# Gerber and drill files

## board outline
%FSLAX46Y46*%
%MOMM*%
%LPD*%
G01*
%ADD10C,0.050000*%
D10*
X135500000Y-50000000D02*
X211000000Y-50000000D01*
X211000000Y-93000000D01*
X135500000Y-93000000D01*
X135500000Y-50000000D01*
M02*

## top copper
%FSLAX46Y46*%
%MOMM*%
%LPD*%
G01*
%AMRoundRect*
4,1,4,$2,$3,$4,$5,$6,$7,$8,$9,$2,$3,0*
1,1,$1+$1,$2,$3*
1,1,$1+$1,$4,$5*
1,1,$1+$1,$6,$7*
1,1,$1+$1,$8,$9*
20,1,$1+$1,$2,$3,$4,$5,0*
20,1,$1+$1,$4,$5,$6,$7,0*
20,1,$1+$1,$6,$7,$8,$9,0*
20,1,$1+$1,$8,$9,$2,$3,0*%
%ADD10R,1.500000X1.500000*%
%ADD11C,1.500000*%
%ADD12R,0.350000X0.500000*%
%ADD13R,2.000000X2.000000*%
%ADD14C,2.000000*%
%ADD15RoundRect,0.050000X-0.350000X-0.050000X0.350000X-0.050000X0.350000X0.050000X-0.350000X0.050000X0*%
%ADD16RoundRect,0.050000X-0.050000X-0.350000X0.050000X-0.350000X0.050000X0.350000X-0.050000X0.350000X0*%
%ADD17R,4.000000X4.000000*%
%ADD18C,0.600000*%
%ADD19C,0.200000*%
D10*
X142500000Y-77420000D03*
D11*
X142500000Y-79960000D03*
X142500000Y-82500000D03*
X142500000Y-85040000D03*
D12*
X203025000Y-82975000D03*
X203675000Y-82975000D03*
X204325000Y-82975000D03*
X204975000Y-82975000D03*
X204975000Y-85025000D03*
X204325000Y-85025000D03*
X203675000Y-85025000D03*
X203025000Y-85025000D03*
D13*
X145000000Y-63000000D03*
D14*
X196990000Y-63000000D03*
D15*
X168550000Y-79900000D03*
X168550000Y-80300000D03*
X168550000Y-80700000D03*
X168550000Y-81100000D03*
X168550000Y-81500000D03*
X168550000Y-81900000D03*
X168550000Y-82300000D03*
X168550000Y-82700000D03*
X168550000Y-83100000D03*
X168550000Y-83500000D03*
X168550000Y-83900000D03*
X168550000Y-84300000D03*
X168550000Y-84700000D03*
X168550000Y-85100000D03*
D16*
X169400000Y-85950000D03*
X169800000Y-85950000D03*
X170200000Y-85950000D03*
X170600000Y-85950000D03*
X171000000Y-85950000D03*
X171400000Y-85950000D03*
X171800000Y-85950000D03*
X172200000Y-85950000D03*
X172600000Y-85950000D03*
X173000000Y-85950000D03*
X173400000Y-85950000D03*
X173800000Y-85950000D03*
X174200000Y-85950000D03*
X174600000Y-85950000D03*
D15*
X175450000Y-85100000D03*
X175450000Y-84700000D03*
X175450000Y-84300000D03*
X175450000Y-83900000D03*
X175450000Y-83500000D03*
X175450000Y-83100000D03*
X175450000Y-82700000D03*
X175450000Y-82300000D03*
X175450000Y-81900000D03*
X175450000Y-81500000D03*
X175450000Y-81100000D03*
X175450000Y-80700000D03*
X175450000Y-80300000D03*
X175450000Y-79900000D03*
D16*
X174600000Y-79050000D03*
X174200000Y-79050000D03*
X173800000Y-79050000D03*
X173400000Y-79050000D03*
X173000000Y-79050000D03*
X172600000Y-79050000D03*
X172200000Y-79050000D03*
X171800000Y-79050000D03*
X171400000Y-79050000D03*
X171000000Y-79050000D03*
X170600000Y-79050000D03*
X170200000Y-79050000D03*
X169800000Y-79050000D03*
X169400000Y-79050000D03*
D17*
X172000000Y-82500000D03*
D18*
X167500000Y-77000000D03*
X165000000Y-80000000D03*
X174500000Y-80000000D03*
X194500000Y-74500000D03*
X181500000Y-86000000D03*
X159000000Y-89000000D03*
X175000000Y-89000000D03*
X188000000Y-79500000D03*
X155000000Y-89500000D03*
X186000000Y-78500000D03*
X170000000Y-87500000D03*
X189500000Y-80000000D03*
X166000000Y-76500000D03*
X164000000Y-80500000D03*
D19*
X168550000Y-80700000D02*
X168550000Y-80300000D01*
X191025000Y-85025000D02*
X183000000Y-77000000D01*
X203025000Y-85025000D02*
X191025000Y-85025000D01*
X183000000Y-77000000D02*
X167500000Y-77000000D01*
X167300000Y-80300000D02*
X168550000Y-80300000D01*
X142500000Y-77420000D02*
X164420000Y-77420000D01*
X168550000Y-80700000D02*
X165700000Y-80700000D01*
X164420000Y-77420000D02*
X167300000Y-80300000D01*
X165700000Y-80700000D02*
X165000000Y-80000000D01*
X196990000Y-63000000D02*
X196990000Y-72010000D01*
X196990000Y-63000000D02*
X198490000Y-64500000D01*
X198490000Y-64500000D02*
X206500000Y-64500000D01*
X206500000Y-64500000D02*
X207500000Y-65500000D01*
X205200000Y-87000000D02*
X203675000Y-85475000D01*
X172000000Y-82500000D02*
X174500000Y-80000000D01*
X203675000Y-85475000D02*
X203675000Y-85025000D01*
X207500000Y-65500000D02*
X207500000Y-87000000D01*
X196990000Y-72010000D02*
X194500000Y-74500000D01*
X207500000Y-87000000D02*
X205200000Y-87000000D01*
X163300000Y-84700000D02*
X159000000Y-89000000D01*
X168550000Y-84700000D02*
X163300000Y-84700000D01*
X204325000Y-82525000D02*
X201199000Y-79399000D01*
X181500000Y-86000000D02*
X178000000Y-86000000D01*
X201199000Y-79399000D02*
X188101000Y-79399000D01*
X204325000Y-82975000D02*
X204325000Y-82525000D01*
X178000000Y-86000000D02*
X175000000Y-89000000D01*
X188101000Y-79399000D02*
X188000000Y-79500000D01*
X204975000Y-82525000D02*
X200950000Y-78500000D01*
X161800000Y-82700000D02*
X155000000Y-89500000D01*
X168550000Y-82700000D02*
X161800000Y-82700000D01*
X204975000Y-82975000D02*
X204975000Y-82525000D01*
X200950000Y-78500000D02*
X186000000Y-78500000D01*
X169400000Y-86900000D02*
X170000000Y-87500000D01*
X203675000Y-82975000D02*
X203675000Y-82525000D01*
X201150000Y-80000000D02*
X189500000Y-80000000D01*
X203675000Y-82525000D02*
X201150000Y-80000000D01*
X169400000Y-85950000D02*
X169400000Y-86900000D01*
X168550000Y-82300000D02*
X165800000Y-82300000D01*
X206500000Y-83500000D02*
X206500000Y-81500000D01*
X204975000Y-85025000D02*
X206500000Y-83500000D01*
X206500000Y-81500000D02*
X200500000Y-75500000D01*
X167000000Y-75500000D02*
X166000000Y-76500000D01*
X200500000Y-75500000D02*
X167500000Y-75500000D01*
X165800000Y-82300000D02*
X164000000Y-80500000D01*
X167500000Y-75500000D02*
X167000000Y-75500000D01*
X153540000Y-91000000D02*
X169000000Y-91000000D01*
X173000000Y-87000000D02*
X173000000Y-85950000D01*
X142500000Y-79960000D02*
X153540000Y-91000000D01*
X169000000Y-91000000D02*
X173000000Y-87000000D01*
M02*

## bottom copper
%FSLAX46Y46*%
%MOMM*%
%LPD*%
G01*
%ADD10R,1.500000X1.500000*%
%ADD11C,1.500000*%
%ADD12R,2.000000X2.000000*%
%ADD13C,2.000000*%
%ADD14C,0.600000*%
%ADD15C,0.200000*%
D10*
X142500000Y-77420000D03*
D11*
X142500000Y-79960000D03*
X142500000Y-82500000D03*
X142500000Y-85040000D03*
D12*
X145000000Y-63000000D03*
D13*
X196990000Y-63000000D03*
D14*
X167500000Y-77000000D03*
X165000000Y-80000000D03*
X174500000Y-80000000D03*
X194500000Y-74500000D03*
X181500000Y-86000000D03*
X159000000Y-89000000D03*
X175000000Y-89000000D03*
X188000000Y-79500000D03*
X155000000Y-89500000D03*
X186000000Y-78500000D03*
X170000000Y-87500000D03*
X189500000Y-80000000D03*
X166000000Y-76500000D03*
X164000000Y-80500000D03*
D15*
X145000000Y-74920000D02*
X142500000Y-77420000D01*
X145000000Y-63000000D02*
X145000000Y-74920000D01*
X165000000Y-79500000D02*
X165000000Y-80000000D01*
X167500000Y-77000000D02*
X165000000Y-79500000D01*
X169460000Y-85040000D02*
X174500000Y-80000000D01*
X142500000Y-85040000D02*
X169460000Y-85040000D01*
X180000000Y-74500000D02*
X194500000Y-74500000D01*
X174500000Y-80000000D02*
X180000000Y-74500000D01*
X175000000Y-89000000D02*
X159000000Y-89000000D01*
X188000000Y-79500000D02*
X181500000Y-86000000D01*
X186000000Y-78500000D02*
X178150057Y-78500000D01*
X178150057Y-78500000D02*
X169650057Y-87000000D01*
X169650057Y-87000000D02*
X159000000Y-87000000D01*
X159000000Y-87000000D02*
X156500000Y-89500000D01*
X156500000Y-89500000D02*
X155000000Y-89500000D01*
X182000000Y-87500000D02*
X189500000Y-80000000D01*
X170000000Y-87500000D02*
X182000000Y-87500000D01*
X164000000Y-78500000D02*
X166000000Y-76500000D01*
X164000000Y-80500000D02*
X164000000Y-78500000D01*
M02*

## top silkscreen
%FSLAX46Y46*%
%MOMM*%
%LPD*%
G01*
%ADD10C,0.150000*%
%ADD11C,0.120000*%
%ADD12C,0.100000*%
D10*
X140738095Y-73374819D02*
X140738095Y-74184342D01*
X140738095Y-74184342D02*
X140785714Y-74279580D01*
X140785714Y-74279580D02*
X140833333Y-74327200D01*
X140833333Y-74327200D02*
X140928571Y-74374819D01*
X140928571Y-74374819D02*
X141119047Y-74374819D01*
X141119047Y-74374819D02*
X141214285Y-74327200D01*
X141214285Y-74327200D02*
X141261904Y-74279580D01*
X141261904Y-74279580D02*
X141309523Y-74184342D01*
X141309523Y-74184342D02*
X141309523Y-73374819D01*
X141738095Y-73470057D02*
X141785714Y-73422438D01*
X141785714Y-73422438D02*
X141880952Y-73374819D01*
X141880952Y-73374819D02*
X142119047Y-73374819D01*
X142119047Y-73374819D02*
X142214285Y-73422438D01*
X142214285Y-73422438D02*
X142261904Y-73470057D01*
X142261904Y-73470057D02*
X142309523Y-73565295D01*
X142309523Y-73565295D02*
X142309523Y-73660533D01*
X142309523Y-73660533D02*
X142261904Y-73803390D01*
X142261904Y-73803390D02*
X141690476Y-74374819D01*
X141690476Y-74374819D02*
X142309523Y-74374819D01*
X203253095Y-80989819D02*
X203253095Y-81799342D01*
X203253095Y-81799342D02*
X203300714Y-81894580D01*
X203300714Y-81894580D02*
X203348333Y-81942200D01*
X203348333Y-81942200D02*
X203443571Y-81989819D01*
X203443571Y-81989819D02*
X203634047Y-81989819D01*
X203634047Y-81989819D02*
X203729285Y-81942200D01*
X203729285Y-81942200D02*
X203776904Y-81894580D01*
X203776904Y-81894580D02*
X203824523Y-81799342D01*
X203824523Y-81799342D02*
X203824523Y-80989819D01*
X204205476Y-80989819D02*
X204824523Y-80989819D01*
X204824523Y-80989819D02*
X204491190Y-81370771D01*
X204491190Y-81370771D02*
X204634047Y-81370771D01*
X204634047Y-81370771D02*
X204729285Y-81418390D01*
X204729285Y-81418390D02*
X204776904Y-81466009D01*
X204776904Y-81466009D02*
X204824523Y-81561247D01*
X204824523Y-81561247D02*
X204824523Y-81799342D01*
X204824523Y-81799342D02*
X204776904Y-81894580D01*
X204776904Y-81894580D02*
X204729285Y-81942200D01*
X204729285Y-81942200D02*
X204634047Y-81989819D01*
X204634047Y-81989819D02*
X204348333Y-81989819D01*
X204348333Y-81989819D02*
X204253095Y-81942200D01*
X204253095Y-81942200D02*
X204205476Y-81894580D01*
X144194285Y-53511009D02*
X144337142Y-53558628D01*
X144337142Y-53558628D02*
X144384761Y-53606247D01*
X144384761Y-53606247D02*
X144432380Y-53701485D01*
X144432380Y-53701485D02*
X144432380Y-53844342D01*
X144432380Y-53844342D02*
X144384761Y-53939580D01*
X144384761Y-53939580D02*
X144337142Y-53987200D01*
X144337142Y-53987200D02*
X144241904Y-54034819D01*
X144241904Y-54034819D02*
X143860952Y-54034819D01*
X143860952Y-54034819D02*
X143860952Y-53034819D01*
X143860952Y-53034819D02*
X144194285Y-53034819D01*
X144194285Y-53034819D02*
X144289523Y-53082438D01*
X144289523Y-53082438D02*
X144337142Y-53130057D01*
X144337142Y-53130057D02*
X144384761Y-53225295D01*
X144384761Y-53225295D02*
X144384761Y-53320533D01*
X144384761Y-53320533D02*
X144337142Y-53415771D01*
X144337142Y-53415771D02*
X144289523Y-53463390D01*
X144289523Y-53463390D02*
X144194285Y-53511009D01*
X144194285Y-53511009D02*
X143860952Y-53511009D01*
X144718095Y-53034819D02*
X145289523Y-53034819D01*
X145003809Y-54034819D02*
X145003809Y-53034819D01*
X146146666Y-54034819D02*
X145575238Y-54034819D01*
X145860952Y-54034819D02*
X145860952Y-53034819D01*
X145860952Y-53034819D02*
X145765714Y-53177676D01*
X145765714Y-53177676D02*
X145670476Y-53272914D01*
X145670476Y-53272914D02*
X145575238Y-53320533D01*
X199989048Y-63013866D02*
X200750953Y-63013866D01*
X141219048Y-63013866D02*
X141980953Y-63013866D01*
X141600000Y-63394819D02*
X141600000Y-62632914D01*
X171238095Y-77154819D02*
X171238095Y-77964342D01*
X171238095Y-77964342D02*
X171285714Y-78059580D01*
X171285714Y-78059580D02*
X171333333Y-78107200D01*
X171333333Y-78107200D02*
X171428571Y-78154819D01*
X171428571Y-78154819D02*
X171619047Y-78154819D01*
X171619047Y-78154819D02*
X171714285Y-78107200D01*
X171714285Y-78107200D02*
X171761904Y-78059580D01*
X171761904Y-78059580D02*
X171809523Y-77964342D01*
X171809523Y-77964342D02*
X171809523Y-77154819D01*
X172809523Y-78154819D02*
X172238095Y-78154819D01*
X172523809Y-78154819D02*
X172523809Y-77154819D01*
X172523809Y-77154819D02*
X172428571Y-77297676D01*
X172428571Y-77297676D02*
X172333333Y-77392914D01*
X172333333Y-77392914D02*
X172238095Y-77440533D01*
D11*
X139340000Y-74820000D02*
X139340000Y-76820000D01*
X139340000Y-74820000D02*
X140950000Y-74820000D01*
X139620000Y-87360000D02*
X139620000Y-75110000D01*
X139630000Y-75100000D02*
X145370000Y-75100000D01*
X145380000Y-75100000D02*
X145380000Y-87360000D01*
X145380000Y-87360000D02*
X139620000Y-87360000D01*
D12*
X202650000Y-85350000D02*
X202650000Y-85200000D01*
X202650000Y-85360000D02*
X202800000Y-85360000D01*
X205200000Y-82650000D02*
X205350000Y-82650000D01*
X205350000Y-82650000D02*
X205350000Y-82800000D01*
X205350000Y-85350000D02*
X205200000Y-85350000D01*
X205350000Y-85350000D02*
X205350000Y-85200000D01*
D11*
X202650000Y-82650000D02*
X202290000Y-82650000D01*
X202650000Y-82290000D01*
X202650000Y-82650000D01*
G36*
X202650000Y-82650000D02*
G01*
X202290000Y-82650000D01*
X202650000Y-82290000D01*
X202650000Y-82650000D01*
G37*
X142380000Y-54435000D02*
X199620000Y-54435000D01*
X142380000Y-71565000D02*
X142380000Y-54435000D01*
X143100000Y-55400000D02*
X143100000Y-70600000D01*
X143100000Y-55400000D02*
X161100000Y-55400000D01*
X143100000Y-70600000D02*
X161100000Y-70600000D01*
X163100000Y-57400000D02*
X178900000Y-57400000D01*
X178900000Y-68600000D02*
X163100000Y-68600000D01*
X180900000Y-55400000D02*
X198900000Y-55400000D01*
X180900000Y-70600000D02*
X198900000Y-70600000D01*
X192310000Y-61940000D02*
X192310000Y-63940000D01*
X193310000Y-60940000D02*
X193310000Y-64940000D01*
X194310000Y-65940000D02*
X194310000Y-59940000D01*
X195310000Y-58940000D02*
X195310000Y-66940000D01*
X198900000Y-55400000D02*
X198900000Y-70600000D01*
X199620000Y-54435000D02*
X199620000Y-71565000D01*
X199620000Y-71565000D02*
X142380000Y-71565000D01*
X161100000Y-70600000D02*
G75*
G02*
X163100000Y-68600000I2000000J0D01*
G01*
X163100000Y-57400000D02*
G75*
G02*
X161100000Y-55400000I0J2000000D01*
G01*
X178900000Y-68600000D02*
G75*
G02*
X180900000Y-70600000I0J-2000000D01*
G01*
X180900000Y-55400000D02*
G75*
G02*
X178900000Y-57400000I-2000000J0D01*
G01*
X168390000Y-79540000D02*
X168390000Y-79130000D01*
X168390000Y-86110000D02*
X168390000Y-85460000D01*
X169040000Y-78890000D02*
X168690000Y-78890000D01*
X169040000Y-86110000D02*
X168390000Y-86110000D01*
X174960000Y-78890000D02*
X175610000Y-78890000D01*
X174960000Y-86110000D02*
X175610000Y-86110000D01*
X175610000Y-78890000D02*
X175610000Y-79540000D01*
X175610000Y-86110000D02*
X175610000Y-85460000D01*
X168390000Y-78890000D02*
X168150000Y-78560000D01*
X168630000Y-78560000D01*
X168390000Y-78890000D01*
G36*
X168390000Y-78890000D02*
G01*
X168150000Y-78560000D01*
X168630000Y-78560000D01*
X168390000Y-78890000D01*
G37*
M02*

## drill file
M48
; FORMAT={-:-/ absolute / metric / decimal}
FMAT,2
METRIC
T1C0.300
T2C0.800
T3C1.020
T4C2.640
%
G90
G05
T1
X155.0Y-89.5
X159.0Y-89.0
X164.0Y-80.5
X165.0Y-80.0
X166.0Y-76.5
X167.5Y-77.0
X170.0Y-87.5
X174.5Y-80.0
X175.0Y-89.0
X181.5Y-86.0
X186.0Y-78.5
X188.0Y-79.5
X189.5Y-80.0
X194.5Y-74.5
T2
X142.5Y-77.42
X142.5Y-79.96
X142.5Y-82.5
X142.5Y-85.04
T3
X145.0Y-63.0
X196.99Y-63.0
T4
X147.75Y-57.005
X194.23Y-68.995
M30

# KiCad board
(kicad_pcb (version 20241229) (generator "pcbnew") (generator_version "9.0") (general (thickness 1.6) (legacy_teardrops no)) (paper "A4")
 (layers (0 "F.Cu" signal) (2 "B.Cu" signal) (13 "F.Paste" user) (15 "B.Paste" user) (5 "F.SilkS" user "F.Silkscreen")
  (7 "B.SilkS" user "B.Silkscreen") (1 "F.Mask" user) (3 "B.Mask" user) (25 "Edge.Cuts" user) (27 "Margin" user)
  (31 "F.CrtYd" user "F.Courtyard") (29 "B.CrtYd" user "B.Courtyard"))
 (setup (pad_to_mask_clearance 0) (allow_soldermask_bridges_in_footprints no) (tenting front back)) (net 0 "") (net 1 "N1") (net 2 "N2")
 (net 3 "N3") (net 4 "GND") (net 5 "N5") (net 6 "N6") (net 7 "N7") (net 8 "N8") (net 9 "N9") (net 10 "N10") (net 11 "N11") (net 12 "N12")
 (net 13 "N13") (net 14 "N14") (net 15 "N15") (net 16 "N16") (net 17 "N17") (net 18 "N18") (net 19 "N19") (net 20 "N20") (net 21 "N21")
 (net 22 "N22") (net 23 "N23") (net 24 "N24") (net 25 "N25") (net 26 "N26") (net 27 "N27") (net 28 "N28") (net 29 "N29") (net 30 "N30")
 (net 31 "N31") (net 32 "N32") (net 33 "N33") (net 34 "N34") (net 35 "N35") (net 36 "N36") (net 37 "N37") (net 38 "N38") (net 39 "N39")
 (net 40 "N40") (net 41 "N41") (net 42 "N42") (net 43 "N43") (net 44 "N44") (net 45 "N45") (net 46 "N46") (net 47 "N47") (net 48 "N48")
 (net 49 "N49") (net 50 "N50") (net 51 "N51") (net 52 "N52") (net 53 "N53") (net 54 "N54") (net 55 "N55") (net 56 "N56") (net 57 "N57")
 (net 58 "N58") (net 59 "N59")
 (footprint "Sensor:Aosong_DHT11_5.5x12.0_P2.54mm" (layer "F.Cu") (at 142.5 77.42)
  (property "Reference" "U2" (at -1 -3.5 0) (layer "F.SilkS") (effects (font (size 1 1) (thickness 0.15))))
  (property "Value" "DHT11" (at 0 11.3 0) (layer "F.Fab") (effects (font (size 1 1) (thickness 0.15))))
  (fp_line (start -3.16 -2.6) (end -3.16 -0.6) (stroke (width 0.12) (type solid)) (layer "F.SilkS"))
  (fp_line (start -3.16 -2.6) (end -1.55 -2.6) (stroke (width 0.12) (type solid)) (layer "F.SilkS"))
  (fp_line (start -2.88 9.94) (end -2.88 -2.31) (stroke (width 0.12) (type solid)) (layer "F.SilkS"))
  (fp_line (start -2.87 -2.32) (end 2.87 -2.32) (stroke (width 0.12) (type solid)) (layer "F.SilkS"))
  (fp_line (start 2.88 -2.32) (end 2.88 9.94) (stroke (width 0.12) (type solid)) (layer "F.SilkS"))
  (fp_line (start 2.88 9.94) (end -2.88 9.94) (stroke (width 0.12) (type solid)) (layer "F.SilkS"))
  (pad "1" thru_hole rect (at 0 0) (size 1.5 1.5) (drill 0.8) (layers "*.Cu" "*.Mask") (remove_unused_layers no) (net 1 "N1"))
  (pad "2" thru_hole circle (at 0 2.54) (size 1.5 1.5) (drill 0.8) (layers "*.Cu" "*.Mask") (remove_unused_layers no) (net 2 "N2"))
  (pad "3" thru_hole circle (at 0 5.08) (size 1.5 1.5) (drill 0.8) (layers "*.Cu" "*.Mask") (remove_unused_layers no) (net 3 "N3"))
  (pad "4" thru_hole circle (at 0 7.62) (size 1.5 1.5) (drill 0.8) (layers "*.Cu" "*.Mask") (remove_unused_layers no) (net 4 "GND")))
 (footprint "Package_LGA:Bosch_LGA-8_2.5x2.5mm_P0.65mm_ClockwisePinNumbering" (layer "F.Cu") (at 204 84)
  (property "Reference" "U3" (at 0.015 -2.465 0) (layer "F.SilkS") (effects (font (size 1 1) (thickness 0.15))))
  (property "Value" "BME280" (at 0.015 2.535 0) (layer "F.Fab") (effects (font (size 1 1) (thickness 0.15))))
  (fp_line (start -1.35 1.35) (end -1.35 1.2) (stroke (width 0.1) (type solid)) (layer "F.SilkS"))
  (fp_line (start -1.35 1.36) (end -1.2 1.36) (stroke (width 0.1) (type solid)) (layer "F.SilkS"))
  (fp_line (start 1.2 -1.35) (end 1.35 -1.35) (stroke (width 0.1) (type solid)) (layer "F.SilkS"))
  (fp_line (start 1.35 -1.35) (end 1.35 -1.2) (stroke (width 0.1) (type solid)) (layer "F.SilkS"))
  (fp_line (start 1.35 1.35) (end 1.2 1.35) (stroke (width 0.1) (type solid)) (layer "F.SilkS"))
  (fp_line (start 1.35 1.35) (end 1.35 1.2) (stroke (width 0.1) (type solid)) (layer "F.SilkS"))
  (fp_poly
   (pts (xy -1.35 -1.35) (xy -1.71 -1.35) (xy -1.35 -1.71) (xy -1.35 -1.35)) (stroke (width 0.12) (type solid)) (fill yes) (layer "F.SilkS"))
  (pad "1" smd rect (at -0.975 -1.025 90) (size 0.5 0.35) (layers "F.Cu" "F.Mask" "F.Paste") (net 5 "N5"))
  (pad "2" smd rect (at -0.325 -1.025 90) (size 0.5 0.35) (layers "F.Cu" "F.Mask" "F.Paste") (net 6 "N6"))
  (pad "3" smd rect (at 0.325 -1.025 90) (size 0.5 0.35) (layers "F.Cu" "F.Mask" "F.Paste") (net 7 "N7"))
  (pad "4" smd rect (at 0.975 -1.025 90) (size 0.5 0.35) (layers "F.Cu" "F.Mask" "F.Paste") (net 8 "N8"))
  (pad "5" smd rect (at 0.975 1.025 90) (size 0.5 0.35) (layers "F.Cu" "F.Mask" "F.Paste") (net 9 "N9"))
  (pad "6" smd rect (at 0.325 1.025 90) (size 0.5 0.35) (layers "F.Cu" "F.Mask" "F.Paste") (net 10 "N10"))
  (pad "7" smd rect (at -0.325 1.025 90) (size 0.5 0.35) (layers "F.Cu" "F.Mask" "F.Paste") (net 4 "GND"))
  (pad "8" smd rect (at -0.975 1.025 90) (size 0.5 0.35) (layers "F.Cu" "F.Mask" "F.Paste") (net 1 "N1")))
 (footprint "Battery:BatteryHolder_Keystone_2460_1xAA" (layer "F.Cu") (at 145 63)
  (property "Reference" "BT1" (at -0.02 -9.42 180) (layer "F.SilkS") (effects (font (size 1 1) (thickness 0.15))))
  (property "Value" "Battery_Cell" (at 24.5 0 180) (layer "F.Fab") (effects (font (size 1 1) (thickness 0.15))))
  (fp_line (start -2.62 -8.565) (end 54.62 -8.565) (stroke (width 0.12) (type solid)) (layer "F.SilkS"))
  (fp_line (start -2.62 8.565) (end -2.62 -8.565) (stroke (width 0.12) (type solid)) (layer "F.SilkS"))
  (fp_line (start -1.9 -7.6) (end -1.9 7.6) (stroke (width 0.12) (type solid)) (layer "F.SilkS"))
  (fp_line (start -1.9 -7.6) (end 16.1 -7.6) (stroke (width 0.12) (type solid)) (layer "F.SilkS"))
  (fp_line (start -1.9 7.6) (end 16.1 7.6) (stroke (width 0.12) (type solid)) (layer "F.SilkS"))
  (fp_line (start 18.1 -5.6) (end 33.9 -5.6) (stroke (width 0.12) (type solid)) (layer "F.SilkS"))
  (fp_line (start 33.9 5.6) (end 18.1 5.6) (stroke (width 0.12) (type solid)) (layer "F.SilkS"))
  (fp_line (start 35.9 -7.6) (end 53.9 -7.6) (stroke (width 0.12) (type solid)) (layer "F.SilkS"))
  (fp_line (start 35.9 7.6) (end 53.9 7.6) (stroke (width 0.12) (type solid)) (layer "F.SilkS"))
  (fp_line (start 47.31 -1.06) (end 47.31 0.94) (stroke (width 0.12) (type solid)) (layer "F.SilkS"))
  (fp_line (start 48.31 -2.06) (end 48.31 1.94) (stroke (width 0.12) (type solid)) (layer "F.SilkS"))
  (fp_line (start 49.31 2.94) (end 49.31 -3.06) (stroke (width 0.12) (type solid)) (layer "F.SilkS"))
  (fp_line (start 50.31 -4.06) (end 50.31 3.94) (stroke (width 0.12) (type solid)) (layer "F.SilkS"))
  (fp_line (start 53.9 -7.6) (end 53.9 7.6) (stroke (width 0.12) (type solid)) (layer "F.SilkS"))
  (fp_line (start 54.62 -8.565) (end 54.62 8.565) (stroke (width 0.12) (type solid)) (layer "F.SilkS"))
  (fp_line (start 54.62 8.565) (end -2.62 8.565) (stroke (width 0.12) (type solid)) (layer "F.SilkS"))
  (fp_arc (start 16.1 7.6) (mid 16.685786 6.185786) (end 18.1 5.6) (stroke (width 0.12) (type solid)) (layer "F.SilkS"))
  (fp_arc (start 18.1 -5.6) (mid 16.685786 -6.185786) (end 16.1 -7.6) (stroke (width 0.12) (type solid)) (layer "F.SilkS"))
  (fp_arc (start 33.9 5.6) (mid 35.314214 6.185786) (end 35.9 7.6) (stroke (width 0.12) (type solid)) (layer "F.SilkS"))
  (fp_arc (start 35.9 -7.6) (mid 35.314214 -6.185786) (end 33.9 -5.6) (stroke (width 0.12) (type solid)) (layer "F.SilkS"))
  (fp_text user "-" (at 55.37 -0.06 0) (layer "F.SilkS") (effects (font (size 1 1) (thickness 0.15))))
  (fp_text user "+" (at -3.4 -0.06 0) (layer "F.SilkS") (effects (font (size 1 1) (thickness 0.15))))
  (pad "" np_thru_hole circle (at 2.75 -5.995 90) (size 2.64 2.64) (drill 2.64) (layers "*.Cu" "*.Mask"))
  (pad "" np_thru_hole circle (at 49.23 5.995) (size 2.64 2.64) (drill 2.64) (layers "*.Cu" "*.Mask"))
  (pad "1" thru_hole rect (at 0 0 180) (size 2 2) (drill 1.02) (layers "*.Cu" "*.Mask") (remove_unused_layers no) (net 1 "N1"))
  (pad "2" thru_hole circle (at 51.99 0 180) (size 2 2) (drill 1.02) (layers "*.Cu" "*.Mask") (remove_unused_layers no) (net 4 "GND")))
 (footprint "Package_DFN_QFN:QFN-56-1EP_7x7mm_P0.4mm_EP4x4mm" (layer "F.Cu") (at 172 82.5)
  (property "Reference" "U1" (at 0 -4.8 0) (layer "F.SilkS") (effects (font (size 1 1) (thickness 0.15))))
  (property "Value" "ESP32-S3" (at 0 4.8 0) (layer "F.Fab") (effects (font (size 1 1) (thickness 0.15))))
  (fp_line (start -3.61 -2.96) (end -3.61 -3.37) (stroke (width 0.12) (type solid)) (layer "F.SilkS"))
  (fp_line (start -3.61 3.61) (end -3.61 2.96) (stroke (width 0.12) (type solid)) (layer "F.SilkS"))
  (fp_line (start -2.96 -3.61) (end -3.31 -3.61) (stroke (width 0.12) (type solid)) (layer "F.SilkS"))
  (fp_line (start -2.96 3.61) (end -3.61 3.61) (stroke (width 0.12) (type solid)) (layer "F.SilkS"))
  (fp_line (start 2.96 -3.61) (end 3.61 -3.61) (stroke (width 0.12) (type solid)) (layer "F.SilkS"))
  (fp_line (start 2.96 3.61) (end 3.61 3.61) (stroke (width 0.12) (type solid)) (layer "F.SilkS"))
  (fp_line (start 3.61 -3.61) (end 3.61 -2.96) (stroke (width 0.12) (type solid)) (layer "F.SilkS"))
  (fp_line (start 3.61 3.61) (end 3.61 2.96) (stroke (width 0.12) (type solid)) (layer "F.SilkS"))
  (fp_poly
   (pts (xy -3.61 -3.61) (xy -3.85 -3.94) (xy -3.37 -3.94) (xy -3.61 -3.61)) (stroke (width 0.12) (type solid)) (fill yes) (layer "F.SilkS"))
  (pad "" smd roundrect (at -1.33 -1.33) (size 1.07 1.07) (layers "F.Paste") (roundrect_rratio 0.233645))
  (pad "" smd roundrect (at -1.33 0) (size 1.07 1.07) (layers "F.Paste") (roundrect_rratio 0.233645))
  (pad "" smd roundrect (at -1.33 1.33) (size 1.07 1.07) (layers "F.Paste") (roundrect_rratio 0.233645))
  (pad "" smd roundrect (at 0 -1.33) (size 1.07 1.07) (layers "F.Paste") (roundrect_rratio 0.233645))
  (pad "" smd roundrect (at 0 0) (size 1.07 1.07) (layers "F.Paste") (roundrect_rratio 0.233645))
  (pad "" smd roundrect (at 0 1.33) (size 1.07 1.07) (layers "F.Paste") (roundrect_rratio 0.233645))
  (pad "" smd roundrect (at 1.33 -1.33) (size 1.07 1.07) (layers "F.Paste") (roundrect_rratio 0.233645))
  (pad "" smd roundrect (at 1.33 0) (size 1.07 1.07) (layers "F.Paste") (roundrect_rratio 0.233645))
  (pad "" smd roundrect (at 1.33 1.33) (size 1.07 1.07) (layers "F.Paste") (roundrect_rratio 0.233645))
  (pad "1" smd roundrect (at -3.45 -2.6) (size 0.8 0.2) (layers "F.Cu" "F.Mask" "F.Paste") (roundrect_rratio 0.25) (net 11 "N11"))
  (pad "2" smd roundrect (at -3.45 -2.2) (size 0.8 0.2) (layers "F.Cu" "F.Mask" "F.Paste") (roundrect_rratio 0.25) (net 1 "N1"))
  (pad "3" smd roundrect (at -3.45 -1.8) (size 0.8 0.2) (layers "F.Cu" "F.Mask" "F.Paste") (roundrect_rratio 0.25) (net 1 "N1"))
  (pad "4" smd roundrect (at -3.45 -1.4) (size 0.8 0.2) (layers "F.Cu" "F.Mask" "F.Paste") (roundrect_rratio 0.25) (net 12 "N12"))
  (pad "5" smd roundrect (at -3.45 -1) (size 0.8 0.2) (layers "F.Cu" "F.Mask" "F.Paste") (roundrect_rratio 0.25) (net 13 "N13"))
  (pad "6" smd roundrect (at -3.45 -0.6) (size 0.8 0.2) (layers "F.Cu" "F.Mask" "F.Paste") (roundrect_rratio 0.25) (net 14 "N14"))
  (pad "7" smd roundrect (at -3.45 -0.2) (size 0.8 0.2) (layers "F.Cu" "F.Mask" "F.Paste") (roundrect_rratio 0.25) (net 9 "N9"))
  (pad "8" smd roundrect (at -3.45 0.2) (size 0.8 0.2) (layers "F.Cu" "F.Mask" "F.Paste") (roundrect_rratio 0.25) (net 8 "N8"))
  (pad "9" smd roundrect (at -3.45 0.6) (size 0.8 0.2) (layers "F.Cu" "F.Mask" "F.Paste") (roundrect_rratio 0.25) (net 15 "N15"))
  (pad "10" smd roundrect (at -3.45 1) (size 0.8 0.2) (layers "F.Cu" "F.Mask" "F.Paste") (roundrect_rratio 0.25) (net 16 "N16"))
  (pad "11" smd roundrect (at -3.45 1.4) (size 0.8 0.2) (layers "F.Cu" "F.Mask" "F.Paste") (roundrect_rratio 0.25) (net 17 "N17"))
  (pad "12" smd roundrect (at -3.45 1.8) (size 0.8 0.2) (layers "F.Cu" "F.Mask" "F.Paste") (roundrect_rratio 0.25) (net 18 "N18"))
  (pad "13" smd roundrect (at -3.45 2.2) (size 0.8 0.2) (layers "F.Cu" "F.Mask" "F.Paste") (roundrect_rratio 0.25) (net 7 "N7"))
  (pad "14" smd roundrect (at -3.45 2.6) (size 0.8 0.2) (layers "F.Cu" "F.Mask" "F.Paste") (roundrect_rratio 0.25) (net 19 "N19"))
  (pad "15" smd roundrect (at -2.6 3.45) (size 0.2 0.8) (layers "F.Cu" "F.Mask" "F.Paste") (roundrect_rratio 0.25) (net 6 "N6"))
  (pad "16" smd roundrect (at -2.2 3.45) (size 0.2 0.8) (layers "F.Cu" "F.Mask" "F.Paste") (roundrect_rratio 0.25) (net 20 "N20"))
  (pad "17" smd roundrect (at -1.8 3.45) (size 0.2 0.8) (layers "F.Cu" "F.Mask" "F.Paste") (roundrect_rratio 0.25) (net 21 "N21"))
  (pad "18" smd roundrect (at -1.4 3.45) (size 0.2 0.8) (layers "F.Cu" "F.Mask" "F.Paste") (roundrect_rratio 0.25) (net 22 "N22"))
  (pad "19" smd roundrect (at -1 3.45) (size 0.2 0.8) (layers "F.Cu" "F.Mask" "F.Paste") (roundrect_rratio 0.25) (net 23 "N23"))
  (pad "20" smd roundrect (at -0.6 3.45) (size 0.2 0.8) (layers "F.Cu" "F.Mask" "F.Paste") (roundrect_rratio 0.25) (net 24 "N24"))
  (pad "21" smd roundrect (at -0.2 3.45) (size 0.2 0.8) (layers "F.Cu" "F.Mask" "F.Paste") (roundrect_rratio 0.25) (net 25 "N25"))
  (pad "22" smd roundrect (at 0.2 3.45) (size 0.2 0.8) (layers "F.Cu" "F.Mask" "F.Paste") (roundrect_rratio 0.25) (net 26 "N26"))
  (pad "23" smd roundrect (at 0.6 3.45) (size 0.2 0.8) (layers "F.Cu" "F.Mask" "F.Paste") (roundrect_rratio 0.25) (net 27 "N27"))
  (pad "24" smd roundrect (at 1 3.45) (size 0.2 0.8) (layers "F.Cu" "F.Mask" "F.Paste") (roundrect_rratio 0.25) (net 2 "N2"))
  (pad "25" smd roundrect (at 1.4 3.45) (size 0.2 0.8) (layers "F.Cu" "F.Mask" "F.Paste") (roundrect_rratio 0.25) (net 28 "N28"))
  (pad "26" smd roundrect (at 1.8 3.45) (size 0.2 0.8) (layers "F.Cu" "F.Mask" "F.Paste") (roundrect_rratio 0.25) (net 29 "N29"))
  (pad "27" smd roundrect (at 2.2 3.45) (size 0.2 0.8) (layers "F.Cu" "F.Mask" "F.Paste") (roundrect_rratio 0.25) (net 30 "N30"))
  (pad "28" smd roundrect (at 2.6 3.45) (size 0.2 0.8) (layers "F.Cu" "F.Mask" "F.Paste") (roundrect_rratio 0.25) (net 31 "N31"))
  (pad "29" smd roundrect (at 3.45 2.6) (size 0.8 0.2) (layers "F.Cu" "F.Mask" "F.Paste") (roundrect_rratio 0.25) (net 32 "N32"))
  (pad "30" smd roundrect (at 3.45 2.2) (size 0.8 0.2) (layers "F.Cu" "F.Mask" "F.Paste") (roundrect_rratio 0.25) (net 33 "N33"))
  (pad "31" smd roundrect (at 3.45 1.8) (size 0.8 0.2) (layers "F.Cu" "F.Mask" "F.Paste") (roundrect_rratio 0.25) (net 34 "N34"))
  (pad "32" smd roundrect (at 3.45 1.4) (size 0.8 0.2) (layers "F.Cu" "F.Mask" "F.Paste") (roundrect_rratio 0.25) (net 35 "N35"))
  (pad "33" smd roundrect (at 3.45 1) (size 0.8 0.2) (layers "F.Cu" "F.Mask" "F.Paste") (roundrect_rratio 0.25) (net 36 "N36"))
  (pad "34" smd roundrect (at 3.45 0.6) (size 0.8 0.2) (layers "F.Cu" "F.Mask" "F.Paste") (roundrect_rratio 0.25) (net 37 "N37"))
  (pad "35" smd roundrect (at 3.45 0.2) (size 0.8 0.2) (layers "F.Cu" "F.Mask" "F.Paste") (roundrect_rratio 0.25) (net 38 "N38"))
  (pad "36" smd roundrect (at 3.45 -0.2) (size 0.8 0.2) (layers "F.Cu" "F.Mask" "F.Paste") (roundrect_rratio 0.25) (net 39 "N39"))
  (pad "37" smd roundrect (at 3.45 -0.6) (size 0.8 0.2) (layers "F.Cu" "F.Mask" "F.Paste") (roundrect_rratio 0.25) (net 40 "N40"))
  (pad "38" smd roundrect (at 3.45 -1) (size 0.8 0.2) (layers "F.Cu" "F.Mask" "F.Paste") (roundrect_rratio 0.25) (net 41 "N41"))
  (pad "39" smd roundrect (at 3.45 -1.4) (size 0.8 0.2) (layers "F.Cu" "F.Mask" "F.Paste") (roundrect_rratio 0.25) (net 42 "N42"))
  (pad "40" smd roundrect (at 3.45 -1.8) (size 0.8 0.2) (layers "F.Cu" "F.Mask" "F.Paste") (roundrect_rratio 0.25) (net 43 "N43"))
  (pad "41" smd roundrect (at 3.45 -2.2) (size 0.8 0.2) (layers "F.Cu" "F.Mask" "F.Paste") (roundrect_rratio 0.25) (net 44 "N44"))
  (pad "42" smd roundrect (at 3.45 -2.6) (size 0.8 0.2) (layers "F.Cu" "F.Mask" "F.Paste") (roundrect_rratio 0.25) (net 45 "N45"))
  (pad "43" smd roundrect (at 2.6 -3.45) (size 0.2 0.8) (layers "F.Cu" "F.Mask" "F.Paste") (roundrect_rratio 0.25) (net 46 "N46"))
  (pad "44" smd roundrect (at 2.2 -3.45) (size 0.2 0.8) (layers "F.Cu" "F.Mask" "F.Paste") (roundrect_rratio 0.25) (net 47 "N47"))
  (pad "45" smd roundrect (at 1.8 -3.45) (size 0.2 0.8) (layers "F.Cu" "F.Mask" "F.Paste") (roundrect_rratio 0.25) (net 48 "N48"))
  (pad "46" smd roundrect (at 1.4 -3.45) (size 0.2 0.8) (layers "F.Cu" "F.Mask" "F.Paste") (roundrect_rratio 0.25) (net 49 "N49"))
  (pad "47" smd roundrect (at 1 -3.45) (size 0.2 0.8) (layers "F.Cu" "F.Mask" "F.Paste") (roundrect_rratio 0.25) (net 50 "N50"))
  (pad "48" smd roundrect (at 0.6 -3.45) (size 0.2 0.8) (layers "F.Cu" "F.Mask" "F.Paste") (roundrect_rratio 0.25) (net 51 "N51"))
  (pad "49" smd roundrect (at 0.2 -3.45) (size 0.2 0.8) (layers "F.Cu" "F.Mask" "F.Paste") (roundrect_rratio 0.25) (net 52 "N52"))
  (pad "50" smd roundrect (at -0.2 -3.45) (size 0.2 0.8) (layers "F.Cu" "F.Mask" "F.Paste") (roundrect_rratio 0.25) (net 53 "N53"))
  (pad "51" smd roundrect (at -0.6 -3.45) (size 0.2 0.8) (layers "F.Cu" "F.Mask" "F.Paste") (roundrect_rratio 0.25) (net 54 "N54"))
  (pad "52" smd roundrect (at -1 -3.45) (size 0.2 0.8) (layers "F.Cu" "F.Mask" "F.Paste") (roundrect_rratio 0.25) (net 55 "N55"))
  (pad "53" smd roundrect (at -1.4 -3.45) (size 0.2 0.8) (layers "F.Cu" "F.Mask" "F.Paste") (roundrect_rratio 0.25) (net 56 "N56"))
  (pad "54" smd roundrect (at -1.8 -3.45) (size 0.2 0.8) (layers "F.Cu" "F.Mask" "F.Paste") (roundrect_rratio 0.25) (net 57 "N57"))
  (pad "55" smd roundrect (at -2.2 -3.45) (size 0.2 0.8) (layers "F.Cu" "F.Mask" "F.Paste") (roundrect_rratio 0.25) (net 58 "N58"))
  (pad "56" smd roundrect (at -2.6 -3.45) (size 0.2 0.8) (layers "F.Cu" "F.Mask" "F.Paste") (roundrect_rratio 0.25) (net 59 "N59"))
  (pad "57" smd rect (at 0 0) (size 4 4) (layers "F.Cu" "F.Mask") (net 4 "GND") (zone_connect 2)))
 (gr_rect (start 135.5 50) (end 211 93) (stroke (width 0.05) (type default)) (fill no) (layer "Edge.Cuts"))
 (segment (start 168.55 80.7) (end 168.55 80.3) (width 0.2) (layer "F.Cu") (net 1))
 (segment (start 191.025 85.025) (end 183 77) (width 0.2) (layer "F.Cu") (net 1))
 (segment (start 203.025 85.025) (end 191.025 85.025) (width 0.2) (layer "F.Cu") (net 1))
 (segment (start 183 77) (end 167.5 77) (width 0.2) (layer "F.Cu") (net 1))
 (segment (start 167.3 80.3) (end 168.55 80.3) (width 0.2) (layer "F.Cu") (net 1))
 (segment (start 142.5 77.42) (end 164.42 77.42) (width 0.2) (layer "F.Cu") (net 1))
 (segment (start 168.55 80.7) (end 165.7 80.7) (width 0.2) (layer "F.Cu") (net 1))
 (segment (start 164.42 77.42) (end 167.3 80.3) (width 0.2) (layer "F.Cu") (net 1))
 (segment (start 165.7 80.7) (end 165 80) (width 0.2) (layer "F.Cu") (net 1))
 (via (at 167.5 77) (size 0.6) (drill 0.3) (layers "F.Cu" "B.Cu") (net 1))
 (via (at 165 80) (size 0.6) (drill 0.3) (layers "F.Cu" "B.Cu") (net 1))
 (segment (start 145 74.92) (end 142.5 77.42) (width 0.2) (layer "B.Cu") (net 1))
 (segment (start 145 63) (end 145 74.92) (width 0.2) (layer "B.Cu") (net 1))
 (segment (start 165 79.5) (end 165 80) (width 0.2) (layer "B.Cu") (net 1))
 (segment (start 167.5 77) (end 165 79.5) (width 0.2) (layer "B.Cu") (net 1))
 (segment (start 196.99 63) (end 196.99 72.01) (width 0.2) (layer "F.Cu") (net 4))
 (segment (start 196.99 63) (end 198.49 64.5) (width 0.2) (layer "F.Cu") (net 4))
 (segment (start 198.49 64.5) (end 206.5 64.5) (width 0.2) (layer "F.Cu") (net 4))
 (segment (start 206.5 64.5) (end 207.5 65.5) (width 0.2) (layer "F.Cu") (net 4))
 (segment (start 205.2 87) (end 203.675 85.475) (width 0.2) (layer "F.Cu") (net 4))
 (segment (start 172 82.5) (end 174.5 80) (width 0.2) (layer "F.Cu") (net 4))
 (segment (start 203.675 85.475) (end 203.675 85.025) (width 0.2) (layer "F.Cu") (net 4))
 (segment (start 207.5 65.5) (end 207.5 87) (width 0.2) (layer "F.Cu") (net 4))
 (segment (start 196.99 72.01) (end 194.5 74.5) (width 0.2) (layer "F.Cu") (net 4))
 (segment (start 207.5 87) (end 205.2 87) (width 0.2) (layer "F.Cu") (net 4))
 (via (at 174.5 80) (size 0.6) (drill 0.3) (layers "F.Cu" "B.Cu") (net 4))
 (via (at 194.5 74.5) (size 0.6) (drill 0.3) (layers "F.Cu" "B.Cu") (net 4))
 (segment (start 169.46 85.04) (end 174.5 80) (width 0.2) (layer "B.Cu") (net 4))
 (segment (start 142.5 85.04) (end 169.46 85.04) (width 0.2) (layer "B.Cu") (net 4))
 (segment (start 180 74.5) (end 194.5 74.5) (width 0.2) (layer "B.Cu") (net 4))
 (segment (start 174.5 80) (end 180 74.5) (width 0.2) (layer "B.Cu") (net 4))
 (segment (start 163.3 84.7) (end 159 89) (width 0.2) (layer "F.Cu") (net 7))
 (segment (start 168.55 84.7) (end 163.3 84.7) (width 0.2) (layer "F.Cu") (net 7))
 (segment (start 204.325 82.525) (end 201.199 79.399) (width 0.2) (layer "F.Cu") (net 7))
 (segment (start 181.5 86) (end 178 86) (width 0.2) (layer "F.Cu") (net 7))
 (segment (start 201.199 79.399) (end 188.101 79.399) (width 0.2) (layer "F.Cu") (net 7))
 (segment (start 204.325 82.975) (end 204.325 82.525) (width 0.2) (layer "F.Cu") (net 7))
 (segment (start 178 86) (end 175 89) (width 0.2) (layer "F.Cu") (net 7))
 (segment (start 188.101 79.399) (end 188 79.5) (width 0.2) (layer "F.Cu") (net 7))
 (via (at 181.5 86) (size 0.6) (drill 0.3) (layers "F.Cu" "B.Cu") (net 7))
 (via (at 159 89) (size 0.6) (drill 0.3) (layers "F.Cu" "B.Cu") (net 7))
 (via (at 175 89) (size 0.6) (drill 0.3) (layers "F.Cu" "B.Cu") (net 7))
 (via (at 188 79.5) (size 0.6) (drill 0.3) (layers "F.Cu" "B.Cu") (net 7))
 (segment (start 175 89) (end 159 89) (width 0.2) (layer "B.Cu") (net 7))
 (segment (start 188 79.5) (end 181.5 86) (width 0.2) (layer "B.Cu") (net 7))
 (segment (start 204.975 82.525) (end 200.95 78.5) (width 0.2) (layer "F.Cu") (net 8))
 (segment (start 161.8 82.7) (end 155 89.5) (width 0.2) (layer "F.Cu") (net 8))
 (segment (start 168.55 82.7) (end 161.8 82.7) (width 0.2) (layer "F.Cu") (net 8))
 (segment (start 204.975 82.975) (end 204.975 82.525) (width 0.2) (layer "F.Cu") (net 8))
 (segment (start 200.95 78.5) (end 186 78.5) (width 0.2) (layer "F.Cu") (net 8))
 (via (at 155 89.5) (size 0.6) (drill 0.3) (layers "F.Cu" "B.Cu") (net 8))
 (via (at 186 78.5) (size 0.6) (drill 0.3) (layers "F.Cu" "B.Cu") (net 8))
 (segment (start 186 78.5) (end 178.150057 78.5) (width 0.2) (layer "B.Cu") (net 8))
 (segment (start 178.150057 78.5) (end 169.650057 87) (width 0.2) (layer "B.Cu") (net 8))
 (segment (start 169.650057 87) (end 159 87) (width 0.2) (layer "B.Cu") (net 8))
 (segment (start 159 87) (end 156.5 89.5) (width 0.2) (layer "B.Cu") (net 8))
 (segment (start 156.5 89.5) (end 155 89.5) (width 0.2) (layer "B.Cu") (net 8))
 (segment (start 169.4 86.9) (end 170 87.5) (width 0.2) (layer "F.Cu") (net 6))
 (segment (start 203.675 82.975) (end 203.675 82.525) (width 0.2) (layer "F.Cu") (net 6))
 (segment (start 201.15 80) (end 189.5 80) (width 0.2) (layer "F.Cu") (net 6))
 (segment (start 203.675 82.525) (end 201.15 80) (width 0.2) (layer "F.Cu") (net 6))
 (segment (start 169.4 85.95) (end 169.4 86.9) (width 0.2) (layer "F.Cu") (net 6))
 (via (at 170 87.5) (size 0.6) (drill 0.3) (layers "F.Cu" "B.Cu") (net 6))
 (via (at 189.5 80) (size 0.6) (drill 0.3) (layers "F.Cu" "B.Cu") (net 6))
 (segment (start 182 87.5) (end 189.5 80) (width 0.2) (layer "B.Cu") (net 6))
 (segment (start 170 87.5) (end 182 87.5) (width 0.2) (layer "B.Cu") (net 6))
 (segment (start 168.55 82.3) (end 165.8 82.3) (width 0.2) (layer "F.Cu") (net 9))
 (segment (start 206.5 83.5) (end 206.5 81.5) (width 0.2) (layer "F.Cu") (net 9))
 (segment (start 204.975 85.025) (end 206.5 83.5) (width 0.2) (layer "F.Cu") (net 9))
 (segment (start 206.5 81.5) (end 200.5 75.5) (width 0.2) (layer "F.Cu") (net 9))
 (segment (start 167 75.5) (end 166 76.5) (width 0.2) (layer "F.Cu") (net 9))
 (segment (start 200.5 75.5) (end 167.5 75.5) (width 0.2) (layer "F.Cu") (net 9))
 (segment (start 165.8 82.3) (end 164 80.5) (width 0.2) (layer "F.Cu") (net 9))
 (segment (start 167.5 75.5) (end 167 75.5) (width 0.2) (layer "F.Cu") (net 9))
 (via (at 166 76.5) (size 0.6) (drill 0.3) (layers "F.Cu" "B.Cu") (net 9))
 (via (at 164 80.5) (size 0.6) (drill 0.3) (layers "F.Cu" "B.Cu") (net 9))
 (segment (start 164 78.5) (end 166 76.5) (width 0.2) (layer "B.Cu") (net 9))
 (segment (start 164 80.5) (end 164 78.5) (width 0.2) (layer "B.Cu") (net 9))
 (segment (start 153.54 91) (end 169 91) (width 0.2) (layer "F.Cu") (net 2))
 (segment (start 173 87) (end 173 85.95) (width 0.2) (layer "F.Cu") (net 2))
 (segment (start 142.5 79.96) (end 153.54 91) (width 0.2) (layer "F.Cu") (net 2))
 (segment (start 169 91) (end 173 87) (width 0.2) (layer "F.Cu") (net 2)))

